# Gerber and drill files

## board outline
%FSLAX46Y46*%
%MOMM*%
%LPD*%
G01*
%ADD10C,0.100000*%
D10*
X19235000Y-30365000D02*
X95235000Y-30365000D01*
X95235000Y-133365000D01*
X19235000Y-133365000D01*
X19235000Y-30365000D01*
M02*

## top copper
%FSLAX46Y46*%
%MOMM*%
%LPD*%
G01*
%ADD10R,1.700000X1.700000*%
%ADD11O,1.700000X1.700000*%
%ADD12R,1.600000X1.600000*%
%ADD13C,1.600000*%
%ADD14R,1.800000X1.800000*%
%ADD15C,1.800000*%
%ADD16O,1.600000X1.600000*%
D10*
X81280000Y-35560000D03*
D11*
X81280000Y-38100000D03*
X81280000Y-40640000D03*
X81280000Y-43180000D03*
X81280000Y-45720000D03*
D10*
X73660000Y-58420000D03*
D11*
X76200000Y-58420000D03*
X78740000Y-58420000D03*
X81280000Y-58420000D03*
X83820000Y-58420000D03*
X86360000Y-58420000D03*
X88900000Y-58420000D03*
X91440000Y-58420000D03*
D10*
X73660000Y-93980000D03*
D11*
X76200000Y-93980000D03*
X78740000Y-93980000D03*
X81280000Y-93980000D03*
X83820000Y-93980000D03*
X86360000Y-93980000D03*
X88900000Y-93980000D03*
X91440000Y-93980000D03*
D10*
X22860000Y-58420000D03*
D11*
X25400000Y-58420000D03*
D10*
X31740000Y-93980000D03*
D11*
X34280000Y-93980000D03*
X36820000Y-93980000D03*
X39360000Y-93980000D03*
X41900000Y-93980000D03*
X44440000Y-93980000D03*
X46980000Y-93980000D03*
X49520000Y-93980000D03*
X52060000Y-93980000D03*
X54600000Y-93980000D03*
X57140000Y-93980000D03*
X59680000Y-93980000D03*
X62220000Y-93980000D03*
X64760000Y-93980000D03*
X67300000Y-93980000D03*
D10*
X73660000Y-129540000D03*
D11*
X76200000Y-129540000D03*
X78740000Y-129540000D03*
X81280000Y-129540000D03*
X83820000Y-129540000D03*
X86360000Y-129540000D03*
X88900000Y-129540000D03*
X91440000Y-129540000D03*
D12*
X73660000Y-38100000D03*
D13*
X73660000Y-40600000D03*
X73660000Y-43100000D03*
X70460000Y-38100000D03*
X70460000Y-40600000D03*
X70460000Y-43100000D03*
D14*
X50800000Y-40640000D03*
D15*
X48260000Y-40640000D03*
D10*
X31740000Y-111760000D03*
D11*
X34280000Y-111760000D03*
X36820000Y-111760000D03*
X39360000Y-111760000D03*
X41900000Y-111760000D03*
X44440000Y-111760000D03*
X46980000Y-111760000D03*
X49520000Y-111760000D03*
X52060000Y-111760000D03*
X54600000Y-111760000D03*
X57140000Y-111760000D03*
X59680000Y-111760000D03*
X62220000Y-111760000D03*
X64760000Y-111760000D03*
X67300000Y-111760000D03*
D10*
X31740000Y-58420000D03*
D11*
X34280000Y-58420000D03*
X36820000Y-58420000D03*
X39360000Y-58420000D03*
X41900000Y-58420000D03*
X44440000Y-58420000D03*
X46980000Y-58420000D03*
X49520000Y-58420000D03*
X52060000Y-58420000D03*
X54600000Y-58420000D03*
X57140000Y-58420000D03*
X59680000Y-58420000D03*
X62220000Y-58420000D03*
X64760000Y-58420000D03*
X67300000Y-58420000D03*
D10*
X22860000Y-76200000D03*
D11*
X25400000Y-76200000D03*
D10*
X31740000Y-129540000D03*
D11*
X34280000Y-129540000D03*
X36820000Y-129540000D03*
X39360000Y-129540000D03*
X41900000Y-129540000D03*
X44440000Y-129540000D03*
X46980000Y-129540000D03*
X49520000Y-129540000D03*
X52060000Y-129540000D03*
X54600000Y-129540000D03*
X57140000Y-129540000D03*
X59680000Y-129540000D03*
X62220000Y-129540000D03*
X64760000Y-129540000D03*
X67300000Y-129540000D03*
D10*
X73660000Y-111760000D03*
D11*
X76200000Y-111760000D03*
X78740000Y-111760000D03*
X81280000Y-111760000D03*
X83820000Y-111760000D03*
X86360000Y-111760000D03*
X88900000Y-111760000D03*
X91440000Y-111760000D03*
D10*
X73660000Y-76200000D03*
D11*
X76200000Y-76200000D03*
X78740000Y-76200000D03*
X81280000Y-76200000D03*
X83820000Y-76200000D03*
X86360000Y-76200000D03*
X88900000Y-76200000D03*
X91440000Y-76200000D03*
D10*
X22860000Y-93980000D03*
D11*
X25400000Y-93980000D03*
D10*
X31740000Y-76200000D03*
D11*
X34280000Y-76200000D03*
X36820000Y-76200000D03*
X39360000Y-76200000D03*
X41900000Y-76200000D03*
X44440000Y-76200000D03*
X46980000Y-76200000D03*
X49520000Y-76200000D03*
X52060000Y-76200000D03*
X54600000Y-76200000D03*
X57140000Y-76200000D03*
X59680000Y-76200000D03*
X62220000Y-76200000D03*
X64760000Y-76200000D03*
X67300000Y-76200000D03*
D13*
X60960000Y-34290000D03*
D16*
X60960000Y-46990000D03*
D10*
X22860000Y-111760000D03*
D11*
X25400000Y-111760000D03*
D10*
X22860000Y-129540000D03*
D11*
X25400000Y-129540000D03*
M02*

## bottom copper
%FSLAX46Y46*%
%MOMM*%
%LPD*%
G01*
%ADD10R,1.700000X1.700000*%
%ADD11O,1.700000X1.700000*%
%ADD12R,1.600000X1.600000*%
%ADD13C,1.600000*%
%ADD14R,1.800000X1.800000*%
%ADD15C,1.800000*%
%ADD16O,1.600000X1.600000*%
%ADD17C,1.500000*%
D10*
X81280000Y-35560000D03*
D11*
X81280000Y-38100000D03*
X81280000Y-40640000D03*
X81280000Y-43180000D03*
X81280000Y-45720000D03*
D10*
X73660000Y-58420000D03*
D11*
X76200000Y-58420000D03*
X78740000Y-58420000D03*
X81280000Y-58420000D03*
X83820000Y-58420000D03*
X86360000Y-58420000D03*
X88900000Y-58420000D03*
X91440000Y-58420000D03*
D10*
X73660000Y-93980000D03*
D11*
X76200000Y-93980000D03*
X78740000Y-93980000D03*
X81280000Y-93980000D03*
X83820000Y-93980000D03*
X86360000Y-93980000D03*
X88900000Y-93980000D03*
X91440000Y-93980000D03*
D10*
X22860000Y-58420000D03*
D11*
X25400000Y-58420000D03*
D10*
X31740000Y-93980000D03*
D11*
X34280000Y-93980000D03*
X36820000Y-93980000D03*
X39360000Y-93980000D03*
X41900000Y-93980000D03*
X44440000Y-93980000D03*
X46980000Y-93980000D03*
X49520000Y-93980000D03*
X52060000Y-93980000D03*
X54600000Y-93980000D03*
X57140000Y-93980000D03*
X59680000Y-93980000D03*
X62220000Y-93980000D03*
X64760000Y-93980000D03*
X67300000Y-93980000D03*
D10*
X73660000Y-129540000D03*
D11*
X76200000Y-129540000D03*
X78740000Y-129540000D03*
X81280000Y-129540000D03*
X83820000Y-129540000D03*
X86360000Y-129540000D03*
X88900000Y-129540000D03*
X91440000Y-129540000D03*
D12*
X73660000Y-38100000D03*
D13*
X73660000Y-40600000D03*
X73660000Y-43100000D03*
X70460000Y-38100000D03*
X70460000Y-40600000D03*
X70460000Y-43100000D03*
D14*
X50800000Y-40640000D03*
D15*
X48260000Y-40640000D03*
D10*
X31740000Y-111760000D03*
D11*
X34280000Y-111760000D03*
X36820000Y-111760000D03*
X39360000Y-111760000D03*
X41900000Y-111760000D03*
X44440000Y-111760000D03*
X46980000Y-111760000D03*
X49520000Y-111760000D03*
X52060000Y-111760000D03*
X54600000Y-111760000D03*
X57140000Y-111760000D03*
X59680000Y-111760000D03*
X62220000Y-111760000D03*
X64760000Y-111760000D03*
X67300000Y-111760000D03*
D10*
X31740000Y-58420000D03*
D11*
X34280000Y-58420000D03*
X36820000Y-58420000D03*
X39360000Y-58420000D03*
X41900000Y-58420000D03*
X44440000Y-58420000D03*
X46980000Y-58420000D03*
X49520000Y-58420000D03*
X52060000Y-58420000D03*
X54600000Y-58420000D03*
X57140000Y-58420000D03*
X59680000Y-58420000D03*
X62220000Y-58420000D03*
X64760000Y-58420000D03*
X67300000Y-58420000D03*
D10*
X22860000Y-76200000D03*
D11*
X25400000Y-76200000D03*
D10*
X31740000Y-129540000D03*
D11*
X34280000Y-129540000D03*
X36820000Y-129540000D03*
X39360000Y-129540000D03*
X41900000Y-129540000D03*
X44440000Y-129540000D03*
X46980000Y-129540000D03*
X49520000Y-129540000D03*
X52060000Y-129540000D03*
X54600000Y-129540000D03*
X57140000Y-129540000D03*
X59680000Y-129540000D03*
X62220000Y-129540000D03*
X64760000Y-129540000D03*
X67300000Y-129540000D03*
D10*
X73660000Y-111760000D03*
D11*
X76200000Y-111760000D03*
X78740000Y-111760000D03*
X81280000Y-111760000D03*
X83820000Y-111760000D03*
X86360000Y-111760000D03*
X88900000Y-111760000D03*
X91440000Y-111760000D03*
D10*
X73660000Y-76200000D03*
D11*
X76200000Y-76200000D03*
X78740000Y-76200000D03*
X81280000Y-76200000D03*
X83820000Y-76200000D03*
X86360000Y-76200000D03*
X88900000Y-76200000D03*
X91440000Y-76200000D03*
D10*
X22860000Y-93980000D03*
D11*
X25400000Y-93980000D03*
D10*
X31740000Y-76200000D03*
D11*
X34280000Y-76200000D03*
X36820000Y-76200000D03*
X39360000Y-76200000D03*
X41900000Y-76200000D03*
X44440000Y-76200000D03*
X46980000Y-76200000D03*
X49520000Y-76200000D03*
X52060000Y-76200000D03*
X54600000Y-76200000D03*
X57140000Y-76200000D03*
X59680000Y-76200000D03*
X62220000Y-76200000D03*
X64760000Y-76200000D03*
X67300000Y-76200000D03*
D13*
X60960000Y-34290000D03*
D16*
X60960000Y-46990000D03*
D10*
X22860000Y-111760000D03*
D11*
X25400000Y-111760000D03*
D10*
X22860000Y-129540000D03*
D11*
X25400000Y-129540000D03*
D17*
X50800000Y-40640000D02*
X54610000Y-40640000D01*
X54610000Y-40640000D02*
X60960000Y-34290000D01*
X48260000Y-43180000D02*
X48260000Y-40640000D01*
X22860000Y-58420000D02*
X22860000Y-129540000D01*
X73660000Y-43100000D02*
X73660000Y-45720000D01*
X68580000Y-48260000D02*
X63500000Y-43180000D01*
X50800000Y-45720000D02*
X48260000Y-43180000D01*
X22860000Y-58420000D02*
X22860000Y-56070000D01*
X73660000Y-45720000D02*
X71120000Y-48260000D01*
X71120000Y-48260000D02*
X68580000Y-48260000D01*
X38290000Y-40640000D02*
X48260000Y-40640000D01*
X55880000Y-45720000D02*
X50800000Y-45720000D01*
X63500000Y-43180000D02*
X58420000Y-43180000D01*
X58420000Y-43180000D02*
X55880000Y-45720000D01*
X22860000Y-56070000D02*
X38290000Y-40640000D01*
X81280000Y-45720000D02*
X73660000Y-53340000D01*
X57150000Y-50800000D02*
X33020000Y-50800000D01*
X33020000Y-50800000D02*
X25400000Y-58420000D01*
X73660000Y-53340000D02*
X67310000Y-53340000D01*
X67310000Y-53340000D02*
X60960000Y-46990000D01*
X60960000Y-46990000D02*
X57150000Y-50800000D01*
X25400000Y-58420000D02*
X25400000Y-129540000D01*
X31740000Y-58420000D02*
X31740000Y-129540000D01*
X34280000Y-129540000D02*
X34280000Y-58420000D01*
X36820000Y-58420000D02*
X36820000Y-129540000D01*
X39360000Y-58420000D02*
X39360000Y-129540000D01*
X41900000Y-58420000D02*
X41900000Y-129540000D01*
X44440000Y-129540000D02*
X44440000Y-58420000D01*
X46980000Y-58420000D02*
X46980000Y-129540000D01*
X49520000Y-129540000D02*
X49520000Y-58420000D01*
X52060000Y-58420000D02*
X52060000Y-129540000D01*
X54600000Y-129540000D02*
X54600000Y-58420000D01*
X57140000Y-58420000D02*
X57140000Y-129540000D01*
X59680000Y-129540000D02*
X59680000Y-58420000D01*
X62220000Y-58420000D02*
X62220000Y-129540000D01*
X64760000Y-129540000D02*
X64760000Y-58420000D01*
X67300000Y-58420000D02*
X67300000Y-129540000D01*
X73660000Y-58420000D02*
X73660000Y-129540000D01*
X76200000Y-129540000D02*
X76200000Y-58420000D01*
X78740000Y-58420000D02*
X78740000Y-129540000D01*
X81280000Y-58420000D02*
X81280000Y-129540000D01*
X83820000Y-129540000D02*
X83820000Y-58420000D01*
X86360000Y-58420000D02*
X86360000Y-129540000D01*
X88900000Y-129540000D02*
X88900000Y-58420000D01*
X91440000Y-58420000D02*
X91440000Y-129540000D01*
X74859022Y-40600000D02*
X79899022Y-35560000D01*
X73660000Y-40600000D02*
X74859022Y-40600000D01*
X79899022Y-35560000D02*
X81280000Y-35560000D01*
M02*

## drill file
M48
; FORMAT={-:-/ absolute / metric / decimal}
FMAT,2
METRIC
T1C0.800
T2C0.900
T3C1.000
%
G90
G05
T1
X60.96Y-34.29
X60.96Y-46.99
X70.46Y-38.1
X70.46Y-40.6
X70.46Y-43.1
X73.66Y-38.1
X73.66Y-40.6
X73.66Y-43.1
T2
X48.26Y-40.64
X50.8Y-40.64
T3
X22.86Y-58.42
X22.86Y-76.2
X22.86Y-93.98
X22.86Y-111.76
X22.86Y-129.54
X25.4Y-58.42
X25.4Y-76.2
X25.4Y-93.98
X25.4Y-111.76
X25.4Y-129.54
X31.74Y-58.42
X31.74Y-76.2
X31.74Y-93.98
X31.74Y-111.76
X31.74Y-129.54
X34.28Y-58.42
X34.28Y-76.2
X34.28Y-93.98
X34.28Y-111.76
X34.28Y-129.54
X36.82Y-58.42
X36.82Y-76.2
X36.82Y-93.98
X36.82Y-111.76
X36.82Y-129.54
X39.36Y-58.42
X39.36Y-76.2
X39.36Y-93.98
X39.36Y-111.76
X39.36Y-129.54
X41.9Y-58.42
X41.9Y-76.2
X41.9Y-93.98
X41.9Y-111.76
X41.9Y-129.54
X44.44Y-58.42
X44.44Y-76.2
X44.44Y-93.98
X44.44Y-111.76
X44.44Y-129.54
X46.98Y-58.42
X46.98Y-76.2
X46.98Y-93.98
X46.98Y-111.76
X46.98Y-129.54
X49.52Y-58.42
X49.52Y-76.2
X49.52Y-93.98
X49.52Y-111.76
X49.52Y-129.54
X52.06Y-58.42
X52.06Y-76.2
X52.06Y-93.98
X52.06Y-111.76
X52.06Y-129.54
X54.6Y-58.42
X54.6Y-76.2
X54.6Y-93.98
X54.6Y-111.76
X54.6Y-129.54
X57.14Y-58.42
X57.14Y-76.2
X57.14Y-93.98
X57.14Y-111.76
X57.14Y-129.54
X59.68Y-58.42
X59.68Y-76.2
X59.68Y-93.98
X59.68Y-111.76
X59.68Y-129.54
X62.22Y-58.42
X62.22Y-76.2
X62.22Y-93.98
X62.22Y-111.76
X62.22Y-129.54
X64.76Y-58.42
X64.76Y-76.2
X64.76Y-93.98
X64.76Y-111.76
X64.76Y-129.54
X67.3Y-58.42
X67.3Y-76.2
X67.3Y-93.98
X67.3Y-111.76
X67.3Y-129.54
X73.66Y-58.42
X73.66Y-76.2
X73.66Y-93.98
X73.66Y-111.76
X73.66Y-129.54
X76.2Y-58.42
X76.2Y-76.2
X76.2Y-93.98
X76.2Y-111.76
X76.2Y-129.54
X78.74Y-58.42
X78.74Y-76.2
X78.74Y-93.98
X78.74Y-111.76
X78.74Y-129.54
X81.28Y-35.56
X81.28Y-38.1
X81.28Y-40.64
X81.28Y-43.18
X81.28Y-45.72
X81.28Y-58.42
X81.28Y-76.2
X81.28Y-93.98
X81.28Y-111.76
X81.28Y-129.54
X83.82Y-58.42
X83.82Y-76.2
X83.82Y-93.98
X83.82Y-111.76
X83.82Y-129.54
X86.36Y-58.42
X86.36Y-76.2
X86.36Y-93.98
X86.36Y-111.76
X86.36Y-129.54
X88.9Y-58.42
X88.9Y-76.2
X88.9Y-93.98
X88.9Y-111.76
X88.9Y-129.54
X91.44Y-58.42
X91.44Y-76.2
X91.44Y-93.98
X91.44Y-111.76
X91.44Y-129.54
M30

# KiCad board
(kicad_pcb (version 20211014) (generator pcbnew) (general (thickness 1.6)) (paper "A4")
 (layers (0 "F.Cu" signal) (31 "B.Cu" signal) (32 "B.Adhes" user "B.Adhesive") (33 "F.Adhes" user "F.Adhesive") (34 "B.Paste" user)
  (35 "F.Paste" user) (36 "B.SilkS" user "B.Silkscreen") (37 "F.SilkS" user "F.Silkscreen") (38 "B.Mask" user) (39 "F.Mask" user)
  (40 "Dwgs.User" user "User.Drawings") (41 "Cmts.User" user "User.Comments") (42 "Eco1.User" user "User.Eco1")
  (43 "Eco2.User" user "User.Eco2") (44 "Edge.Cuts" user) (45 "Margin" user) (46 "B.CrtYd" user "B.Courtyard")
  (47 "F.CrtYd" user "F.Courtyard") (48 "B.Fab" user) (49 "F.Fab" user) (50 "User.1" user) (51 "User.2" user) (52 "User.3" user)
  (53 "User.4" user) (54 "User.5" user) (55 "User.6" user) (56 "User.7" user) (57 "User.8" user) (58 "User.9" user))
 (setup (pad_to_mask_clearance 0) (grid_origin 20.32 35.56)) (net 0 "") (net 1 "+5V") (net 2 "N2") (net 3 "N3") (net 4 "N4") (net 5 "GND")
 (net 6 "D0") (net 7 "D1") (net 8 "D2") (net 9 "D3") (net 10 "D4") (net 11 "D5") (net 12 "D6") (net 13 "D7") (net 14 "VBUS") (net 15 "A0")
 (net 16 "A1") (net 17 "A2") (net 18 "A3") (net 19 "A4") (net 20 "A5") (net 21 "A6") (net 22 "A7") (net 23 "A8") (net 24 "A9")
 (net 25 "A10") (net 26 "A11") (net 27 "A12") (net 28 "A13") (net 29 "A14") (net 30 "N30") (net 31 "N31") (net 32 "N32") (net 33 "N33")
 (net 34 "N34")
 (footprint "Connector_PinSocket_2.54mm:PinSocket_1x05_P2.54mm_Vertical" (layer "F.Cu") (at 81.28 35.56)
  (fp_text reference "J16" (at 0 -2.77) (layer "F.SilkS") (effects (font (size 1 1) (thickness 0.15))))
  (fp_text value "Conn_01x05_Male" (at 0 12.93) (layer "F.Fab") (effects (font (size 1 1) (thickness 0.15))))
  (pad "1" thru_hole rect locked (at 0 0) (size 1.7 1.7) (drill 1) (layers *.Cu *.Mask) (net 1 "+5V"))
  (pad "2" thru_hole oval locked (at 0 2.54) (size 1.7 1.7) (drill 1) (layers *.Cu *.Mask) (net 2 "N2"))
  (pad "3" thru_hole oval locked (at 0 5.08) (size 1.7 1.7) (drill 1) (layers *.Cu *.Mask) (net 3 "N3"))
  (pad "4" thru_hole oval locked (at 0 7.62) (size 1.7 1.7) (drill 1) (layers *.Cu *.Mask) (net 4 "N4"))
  (pad "5" thru_hole oval locked (at 0 10.16) (size 1.7 1.7) (drill 1) (layers *.Cu *.Mask) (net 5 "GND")))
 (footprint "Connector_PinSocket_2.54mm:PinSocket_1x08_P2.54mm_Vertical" (layer "F.Cu") (at 73.66 58.42 90)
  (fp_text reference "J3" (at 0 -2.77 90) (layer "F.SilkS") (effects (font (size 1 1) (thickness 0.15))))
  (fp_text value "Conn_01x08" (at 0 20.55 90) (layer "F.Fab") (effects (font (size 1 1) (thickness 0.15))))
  (pad "1" thru_hole rect locked (at 0 0 90) (size 1.7 1.7) (drill 1) (layers *.Cu *.Mask) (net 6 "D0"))
  (pad "2" thru_hole oval locked (at 0 2.54 90) (size 1.7 1.7) (drill 1) (layers *.Cu *.Mask) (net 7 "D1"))
  (pad "3" thru_hole oval locked (at 0 5.08 90) (size 1.7 1.7) (drill 1) (layers *.Cu *.Mask) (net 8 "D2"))
  (pad "4" thru_hole oval locked (at 0 7.62 90) (size 1.7 1.7) (drill 1) (layers *.Cu *.Mask) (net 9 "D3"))
  (pad "5" thru_hole oval locked (at 0 10.16 90) (size 1.7 1.7) (drill 1) (layers *.Cu *.Mask) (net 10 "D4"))
  (pad "6" thru_hole oval locked (at 0 12.7 90) (size 1.7 1.7) (drill 1) (layers *.Cu *.Mask) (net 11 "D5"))
  (pad "7" thru_hole oval locked (at 0 15.24 90) (size 1.7 1.7) (drill 1) (layers *.Cu *.Mask) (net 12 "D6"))
  (pad "8" thru_hole oval locked (at 0 17.78 90) (size 1.7 1.7) (drill 1) (layers *.Cu *.Mask) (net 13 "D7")))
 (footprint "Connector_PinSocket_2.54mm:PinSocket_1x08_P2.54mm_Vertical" (layer "F.Cu") (at 73.66 93.98 90)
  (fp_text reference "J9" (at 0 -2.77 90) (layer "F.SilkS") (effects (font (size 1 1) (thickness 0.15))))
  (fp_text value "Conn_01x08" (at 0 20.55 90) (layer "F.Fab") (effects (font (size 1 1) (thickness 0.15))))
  (pad "1" thru_hole rect locked (at 0 0 90) (size 1.7 1.7) (drill 1) (layers *.Cu *.Mask) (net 6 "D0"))
  (pad "2" thru_hole oval locked (at 0 2.54 90) (size 1.7 1.7) (drill 1) (layers *.Cu *.Mask) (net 7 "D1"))
  (pad "3" thru_hole oval locked (at 0 5.08 90) (size 1.7 1.7) (drill 1) (layers *.Cu *.Mask) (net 8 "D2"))
  (pad "4" thru_hole oval locked (at 0 7.62 90) (size 1.7 1.7) (drill 1) (layers *.Cu *.Mask) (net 9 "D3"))
  (pad "5" thru_hole oval locked (at 0 10.16 90) (size 1.7 1.7) (drill 1) (layers *.Cu *.Mask) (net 10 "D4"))
  (pad "6" thru_hole oval locked (at 0 12.7 90) (size 1.7 1.7) (drill 1) (layers *.Cu *.Mask) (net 11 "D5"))
  (pad "7" thru_hole oval locked (at 0 15.24 90) (size 1.7 1.7) (drill 1) (layers *.Cu *.Mask) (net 12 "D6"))
  (pad "8" thru_hole oval locked (at 0 17.78 90) (size 1.7 1.7) (drill 1) (layers *.Cu *.Mask) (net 13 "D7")))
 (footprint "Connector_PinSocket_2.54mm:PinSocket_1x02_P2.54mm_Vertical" (layer "F.Cu") (at 22.86 58.42 90)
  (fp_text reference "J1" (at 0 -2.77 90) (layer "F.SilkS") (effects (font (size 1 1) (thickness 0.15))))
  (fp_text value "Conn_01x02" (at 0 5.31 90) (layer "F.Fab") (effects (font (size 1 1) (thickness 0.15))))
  (pad "1" thru_hole rect locked (at 0 0 90) (size 1.7 1.7) (drill 1) (layers *.Cu *.Mask) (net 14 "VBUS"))
  (pad "2" thru_hole oval locked (at 0 2.54 90) (size 1.7 1.7) (drill 1) (layers *.Cu *.Mask) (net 5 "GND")))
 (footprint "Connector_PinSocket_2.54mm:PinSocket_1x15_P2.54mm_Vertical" (layer "F.Cu") (at 31.74 93.98 90)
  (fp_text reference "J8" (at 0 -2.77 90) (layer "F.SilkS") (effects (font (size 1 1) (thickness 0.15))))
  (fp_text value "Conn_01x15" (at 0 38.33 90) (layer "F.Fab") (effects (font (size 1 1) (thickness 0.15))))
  (pad "1" thru_hole rect locked (at 0 0 90) (size 1.7 1.7) (drill 1) (layers *.Cu *.Mask) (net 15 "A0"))
  (pad "2" thru_hole oval locked (at 0 2.54 90) (size 1.7 1.7) (drill 1) (layers *.Cu *.Mask) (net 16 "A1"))
  (pad "3" thru_hole oval locked (at 0 5.08 90) (size 1.7 1.7) (drill 1) (layers *.Cu *.Mask) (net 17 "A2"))
  (pad "4" thru_hole oval locked (at 0 7.62 90) (size 1.7 1.7) (drill 1) (layers *.Cu *.Mask) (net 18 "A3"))
  (pad "5" thru_hole oval locked (at 0 10.16 90) (size 1.7 1.7) (drill 1) (layers *.Cu *.Mask) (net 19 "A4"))
  (pad "6" thru_hole oval locked (at 0 12.7 90) (size 1.7 1.7) (drill 1) (layers *.Cu *.Mask) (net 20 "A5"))
  (pad "7" thru_hole oval locked (at 0 15.24 90) (size 1.7 1.7) (drill 1) (layers *.Cu *.Mask) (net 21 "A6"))
  (pad "8" thru_hole oval locked (at 0 17.78 90) (size 1.7 1.7) (drill 1) (layers *.Cu *.Mask) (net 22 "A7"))
  (pad "9" thru_hole oval locked (at 0 20.32 90) (size 1.7 1.7) (drill 1) (layers *.Cu *.Mask) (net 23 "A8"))
  (pad "10" thru_hole oval locked (at 0 22.86 90) (size 1.7 1.7) (drill 1) (layers *.Cu *.Mask) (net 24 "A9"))
  (pad "11" thru_hole oval locked (at 0 25.4 90) (size 1.7 1.7) (drill 1) (layers *.Cu *.Mask) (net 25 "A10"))
  (pad "12" thru_hole oval locked (at 0 27.94 90) (size 1.7 1.7) (drill 1) (layers *.Cu *.Mask) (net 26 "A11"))
  (pad "13" thru_hole oval locked (at 0 30.48 90) (size 1.7 1.7) (drill 1) (layers *.Cu *.Mask) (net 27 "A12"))
  (pad "14" thru_hole oval locked (at 0 33.02 90) (size 1.7 1.7) (drill 1) (layers *.Cu *.Mask) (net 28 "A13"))
  (pad "15" thru_hole oval locked (at 0 35.56 90) (size 1.7 1.7) (drill 1) (layers *.Cu *.Mask) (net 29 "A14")))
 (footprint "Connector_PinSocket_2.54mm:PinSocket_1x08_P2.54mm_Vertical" (layer "F.Cu") (at 73.66 129.54 90)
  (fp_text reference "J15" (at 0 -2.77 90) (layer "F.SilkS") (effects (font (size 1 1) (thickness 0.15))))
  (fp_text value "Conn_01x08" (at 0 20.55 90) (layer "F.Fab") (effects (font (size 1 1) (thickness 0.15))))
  (pad "1" thru_hole rect locked (at 0 0 90) (size 1.7 1.7) (drill 1) (layers *.Cu *.Mask) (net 6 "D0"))
  (pad "2" thru_hole oval locked (at 0 2.54 90) (size 1.7 1.7) (drill 1) (layers *.Cu *.Mask) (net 7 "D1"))
  (pad "3" thru_hole oval locked (at 0 5.08 90) (size 1.7 1.7) (drill 1) (layers *.Cu *.Mask) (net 8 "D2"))
  (pad "4" thru_hole oval locked (at 0 7.62 90) (size 1.7 1.7) (drill 1) (layers *.Cu *.Mask) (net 9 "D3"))
  (pad "5" thru_hole oval locked (at 0 10.16 90) (size 1.7 1.7) (drill 1) (layers *.Cu *.Mask) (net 10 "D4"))
  (pad "6" thru_hole oval locked (at 0 12.7 90) (size 1.7 1.7) (drill 1) (layers *.Cu *.Mask) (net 11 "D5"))
  (pad "7" thru_hole oval locked (at 0 15.24 90) (size 1.7 1.7) (drill 1) (layers *.Cu *.Mask) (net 12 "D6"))
  (pad "8" thru_hole oval locked (at 0 17.78 90) (size 1.7 1.7) (drill 1) (layers *.Cu *.Mask) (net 13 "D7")))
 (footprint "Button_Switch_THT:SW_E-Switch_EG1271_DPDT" (layer "F.Cu") (at 73.66 38.1 -90)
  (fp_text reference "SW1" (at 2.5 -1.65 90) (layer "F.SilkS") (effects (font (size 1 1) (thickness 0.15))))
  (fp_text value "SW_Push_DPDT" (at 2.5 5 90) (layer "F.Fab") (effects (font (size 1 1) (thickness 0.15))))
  (pad "1" thru_hole rect locked (at 0 0 270) (size 1.6 1.6) (drill 0.8) (layers *.Cu *.Mask) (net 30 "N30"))
  (pad "2" thru_hole circle locked (at 2.5 0 270) (size 1.6 1.6) (drill 0.8) (layers *.Cu *.Mask) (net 1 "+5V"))
  (pad "3" thru_hole circle locked (at 5 0 270) (size 1.6 1.6) (drill 0.8) (layers *.Cu *.Mask) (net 14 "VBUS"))
  (pad "4" thru_hole circle locked (at 0 3.2 270) (size 1.6 1.6) (drill 0.8) (layers *.Cu *.Mask) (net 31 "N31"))
  (pad "5" thru_hole circle locked (at 2.5 3.2 270) (size 1.6 1.6) (drill 0.8) (layers *.Cu *.Mask) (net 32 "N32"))
  (pad "6" thru_hole circle locked (at 5 3.2 270) (size 1.6 1.6) (drill 0.8) (layers *.Cu *.Mask) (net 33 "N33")))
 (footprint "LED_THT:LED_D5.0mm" (layer "F.Cu") (at 50.8 40.64 180)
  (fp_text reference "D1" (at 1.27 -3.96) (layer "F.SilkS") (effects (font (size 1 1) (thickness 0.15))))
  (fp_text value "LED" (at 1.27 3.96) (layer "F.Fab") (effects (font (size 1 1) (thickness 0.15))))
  (pad "1" thru_hole rect locked (at 0 0 180) (size 1.8 1.8) (drill 0.9) (layers *.Cu *.Mask) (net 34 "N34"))
  (pad "2" thru_hole circle locked (at 2.54 0 180) (size 1.8 1.8) (drill 0.9) (layers *.Cu *.Mask) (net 14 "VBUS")))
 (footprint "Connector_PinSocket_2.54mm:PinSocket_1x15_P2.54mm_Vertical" (layer "F.Cu") (at 31.74 111.76 90)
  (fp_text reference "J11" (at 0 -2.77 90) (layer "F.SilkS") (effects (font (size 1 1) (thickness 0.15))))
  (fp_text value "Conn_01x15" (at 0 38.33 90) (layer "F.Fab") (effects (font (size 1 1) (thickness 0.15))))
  (pad "1" thru_hole rect locked (at 0 0 90) (size 1.7 1.7) (drill 1) (layers *.Cu *.Mask) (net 15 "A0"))
  (pad "2" thru_hole oval locked (at 0 2.54 90) (size 1.7 1.7) (drill 1) (layers *.Cu *.Mask) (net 16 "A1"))
  (pad "3" thru_hole oval locked (at 0 5.08 90) (size 1.7 1.7) (drill 1) (layers *.Cu *.Mask) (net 17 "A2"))
  (pad "4" thru_hole oval locked (at 0 7.62 90) (size 1.7 1.7) (drill 1) (layers *.Cu *.Mask) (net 18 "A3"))
  (pad "5" thru_hole oval locked (at 0 10.16 90) (size 1.7 1.7) (drill 1) (layers *.Cu *.Mask) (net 19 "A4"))
  (pad "6" thru_hole oval locked (at 0 12.7 90) (size 1.7 1.7) (drill 1) (layers *.Cu *.Mask) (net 20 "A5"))
  (pad "7" thru_hole oval locked (at 0 15.24 90) (size 1.7 1.7) (drill 1) (layers *.Cu *.Mask) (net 21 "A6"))
  (pad "8" thru_hole oval locked (at 0 17.78 90) (size 1.7 1.7) (drill 1) (layers *.Cu *.Mask) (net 22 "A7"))
  (pad "9" thru_hole oval locked (at 0 20.32 90) (size 1.7 1.7) (drill 1) (layers *.Cu *.Mask) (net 23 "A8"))
  (pad "10" thru_hole oval locked (at 0 22.86 90) (size 1.7 1.7) (drill 1) (layers *.Cu *.Mask) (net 24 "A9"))
  (pad "11" thru_hole oval locked (at 0 25.4 90) (size 1.7 1.7) (drill 1) (layers *.Cu *.Mask) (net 25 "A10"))
  (pad "12" thru_hole oval locked (at 0 27.94 90) (size 1.7 1.7) (drill 1) (layers *.Cu *.Mask) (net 26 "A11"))
  (pad "13" thru_hole oval locked (at 0 30.48 90) (size 1.7 1.7) (drill 1) (layers *.Cu *.Mask) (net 27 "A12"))
  (pad "14" thru_hole oval locked (at 0 33.02 90) (size 1.7 1.7) (drill 1) (layers *.Cu *.Mask) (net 28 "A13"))
  (pad "15" thru_hole oval locked (at 0 35.56 90) (size 1.7 1.7) (drill 1) (layers *.Cu *.Mask) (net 29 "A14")))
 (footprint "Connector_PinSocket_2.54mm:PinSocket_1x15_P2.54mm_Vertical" (layer "F.Cu") (at 31.74 58.42 90)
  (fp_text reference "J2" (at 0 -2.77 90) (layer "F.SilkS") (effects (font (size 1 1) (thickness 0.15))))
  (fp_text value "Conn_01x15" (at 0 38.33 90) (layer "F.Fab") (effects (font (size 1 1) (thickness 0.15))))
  (pad "1" thru_hole rect locked (at 0 0 90) (size 1.7 1.7) (drill 1) (layers *.Cu *.Mask) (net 15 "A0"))
  (pad "2" thru_hole oval locked (at 0 2.54 90) (size 1.7 1.7) (drill 1) (layers *.Cu *.Mask) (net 16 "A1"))
  (pad "3" thru_hole oval locked (at 0 5.08 90) (size 1.7 1.7) (drill 1) (layers *.Cu *.Mask) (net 17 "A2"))
  (pad "4" thru_hole oval locked (at 0 7.62 90) (size 1.7 1.7) (drill 1) (layers *.Cu *.Mask) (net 18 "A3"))
  (pad "5" thru_hole oval locked (at 0 10.16 90) (size 1.7 1.7) (drill 1) (layers *.Cu *.Mask) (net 19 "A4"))
  (pad "6" thru_hole oval locked (at 0 12.7 90) (size 1.7 1.7) (drill 1) (layers *.Cu *.Mask) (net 20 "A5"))
  (pad "7" thru_hole oval locked (at 0 15.24 90) (size 1.7 1.7) (drill 1) (layers *.Cu *.Mask) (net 21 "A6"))
  (pad "8" thru_hole oval locked (at 0 17.78 90) (size 1.7 1.7) (drill 1) (layers *.Cu *.Mask) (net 22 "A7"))
  (pad "9" thru_hole oval locked (at 0 20.32 90) (size 1.7 1.7) (drill 1) (layers *.Cu *.Mask) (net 23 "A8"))
  (pad "10" thru_hole oval locked (at 0 22.86 90) (size 1.7 1.7) (drill 1) (layers *.Cu *.Mask) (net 24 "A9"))
  (pad "11" thru_hole oval locked (at 0 25.4 90) (size 1.7 1.7) (drill 1) (layers *.Cu *.Mask) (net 25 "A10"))
  (pad "12" thru_hole oval locked (at 0 27.94 90) (size 1.7 1.7) (drill 1) (layers *.Cu *.Mask) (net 26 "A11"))
  (pad "13" thru_hole oval locked (at 0 30.48 90) (size 1.7 1.7) (drill 1) (layers *.Cu *.Mask) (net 27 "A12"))
  (pad "14" thru_hole oval locked (at 0 33.02 90) (size 1.7 1.7) (drill 1) (layers *.Cu *.Mask) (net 28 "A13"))
  (pad "15" thru_hole oval locked (at 0 35.56 90) (size 1.7 1.7) (drill 1) (layers *.Cu *.Mask) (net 29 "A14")))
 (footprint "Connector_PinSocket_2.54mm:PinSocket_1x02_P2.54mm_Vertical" (layer "F.Cu") (at 22.86 76.2 90)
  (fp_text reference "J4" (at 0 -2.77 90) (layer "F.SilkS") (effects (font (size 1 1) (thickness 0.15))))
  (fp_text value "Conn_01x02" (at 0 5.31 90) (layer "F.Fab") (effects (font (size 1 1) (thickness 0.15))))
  (pad "1" thru_hole rect locked (at 0 0 90) (size 1.7 1.7) (drill 1) (layers *.Cu *.Mask) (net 14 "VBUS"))
  (pad "2" thru_hole oval locked (at 0 2.54 90) (size 1.7 1.7) (drill 1) (layers *.Cu *.Mask) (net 5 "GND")))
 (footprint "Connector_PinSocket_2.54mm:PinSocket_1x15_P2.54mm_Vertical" (layer "F.Cu") (at 31.74 129.54 90)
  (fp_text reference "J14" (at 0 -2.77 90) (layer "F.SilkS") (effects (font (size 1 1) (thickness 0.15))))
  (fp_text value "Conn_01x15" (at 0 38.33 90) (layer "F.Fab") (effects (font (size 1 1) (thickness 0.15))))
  (pad "1" thru_hole rect locked (at 0 0 90) (size 1.7 1.7) (drill 1) (layers *.Cu *.Mask) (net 15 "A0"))
  (pad "2" thru_hole oval locked (at 0 2.54 90) (size 1.7 1.7) (drill 1) (layers *.Cu *.Mask) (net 16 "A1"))
  (pad "3" thru_hole oval locked (at 0 5.08 90) (size 1.7 1.7) (drill 1) (layers *.Cu *.Mask) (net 17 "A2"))
  (pad "4" thru_hole oval locked (at 0 7.62 90) (size 1.7 1.7) (drill 1) (layers *.Cu *.Mask) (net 18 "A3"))
  (pad "5" thru_hole oval locked (at 0 10.16 90) (size 1.7 1.7) (drill 1) (layers *.Cu *.Mask) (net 19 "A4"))
  (pad "6" thru_hole oval locked (at 0 12.7 90) (size 1.7 1.7) (drill 1) (layers *.Cu *.Mask) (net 20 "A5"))
  (pad "7" thru_hole oval locked (at 0 15.24 90) (size 1.7 1.7) (drill 1) (layers *.Cu *.Mask) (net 21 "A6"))
  (pad "8" thru_hole oval locked (at 0 17.78 90) (size 1.7 1.7) (drill 1) (layers *.Cu *.Mask) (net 22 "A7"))
  (pad "9" thru_hole oval locked (at 0 20.32 90) (size 1.7 1.7) (drill 1) (layers *.Cu *.Mask) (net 23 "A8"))
  (pad "10" thru_hole oval locked (at 0 22.86 90) (size 1.7 1.7) (drill 1) (layers *.Cu *.Mask) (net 24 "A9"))
  (pad "11" thru_hole oval locked (at 0 25.4 90) (size 1.7 1.7) (drill 1) (layers *.Cu *.Mask) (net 25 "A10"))
  (pad "12" thru_hole oval locked (at 0 27.94 90) (size 1.7 1.7) (drill 1) (layers *.Cu *.Mask) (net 26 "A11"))
  (pad "13" thru_hole oval locked (at 0 30.48 90) (size 1.7 1.7) (drill 1) (layers *.Cu *.Mask) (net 27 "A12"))
  (pad "14" thru_hole oval locked (at 0 33.02 90) (size 1.7 1.7) (drill 1) (layers *.Cu *.Mask) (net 28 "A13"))
  (pad "15" thru_hole oval locked (at 0 35.56 90) (size 1.7 1.7) (drill 1) (layers *.Cu *.Mask) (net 29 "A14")))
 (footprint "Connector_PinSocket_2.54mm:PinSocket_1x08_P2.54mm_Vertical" (layer "F.Cu") (at 73.66 111.76 90)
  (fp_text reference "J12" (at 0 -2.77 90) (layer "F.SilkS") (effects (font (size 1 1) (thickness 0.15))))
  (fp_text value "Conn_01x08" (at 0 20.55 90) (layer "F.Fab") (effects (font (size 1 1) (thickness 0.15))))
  (pad "1" thru_hole rect locked (at 0 0 90) (size 1.7 1.7) (drill 1) (layers *.Cu *.Mask) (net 6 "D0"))
  (pad "2" thru_hole oval locked (at 0 2.54 90) (size 1.7 1.7) (drill 1) (layers *.Cu *.Mask) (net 7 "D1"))
  (pad "3" thru_hole oval locked (at 0 5.08 90) (size 1.7 1.7) (drill 1) (layers *.Cu *.Mask) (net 8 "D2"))
  (pad "4" thru_hole oval locked (at 0 7.62 90) (size 1.7 1.7) (drill 1) (layers *.Cu *.Mask) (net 9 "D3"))
  (pad "5" thru_hole oval locked (at 0 10.16 90) (size 1.7 1.7) (drill 1) (layers *.Cu *.Mask) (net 10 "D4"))
  (pad "6" thru_hole oval locked (at 0 12.7 90) (size 1.7 1.7) (drill 1) (layers *.Cu *.Mask) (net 11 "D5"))
  (pad "7" thru_hole oval locked (at 0 15.24 90) (size 1.7 1.7) (drill 1) (layers *.Cu *.Mask) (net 12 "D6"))
  (pad "8" thru_hole oval locked (at 0 17.78 90) (size 1.7 1.7) (drill 1) (layers *.Cu *.Mask) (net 13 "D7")))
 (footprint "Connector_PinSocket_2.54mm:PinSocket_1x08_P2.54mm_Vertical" (layer "F.Cu") (at 73.66 76.2 90)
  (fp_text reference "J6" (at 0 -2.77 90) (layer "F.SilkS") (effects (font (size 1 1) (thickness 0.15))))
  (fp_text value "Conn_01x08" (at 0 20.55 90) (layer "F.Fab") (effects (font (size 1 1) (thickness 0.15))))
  (pad "1" thru_hole rect locked (at 0 0 90) (size 1.7 1.7) (drill 1) (layers *.Cu *.Mask) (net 6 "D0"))
  (pad "2" thru_hole oval locked (at 0 2.54 90) (size 1.7 1.7) (drill 1) (layers *.Cu *.Mask) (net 7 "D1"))
  (pad "3" thru_hole oval locked (at 0 5.08 90) (size 1.7 1.7) (drill 1) (layers *.Cu *.Mask) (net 8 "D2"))
  (pad "4" thru_hole oval locked (at 0 7.62 90) (size 1.7 1.7) (drill 1) (layers *.Cu *.Mask) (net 9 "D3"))
  (pad "5" thru_hole oval locked (at 0 10.16 90) (size 1.7 1.7) (drill 1) (layers *.Cu *.Mask) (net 10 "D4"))
  (pad "6" thru_hole oval locked (at 0 12.7 90) (size 1.7 1.7) (drill 1) (layers *.Cu *.Mask) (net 11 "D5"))
  (pad "7" thru_hole oval locked (at 0 15.24 90) (size 1.7 1.7) (drill 1) (layers *.Cu *.Mask) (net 12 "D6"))
  (pad "8" thru_hole oval locked (at 0 17.78 90) (size 1.7 1.7) (drill 1) (layers *.Cu *.Mask) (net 13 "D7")))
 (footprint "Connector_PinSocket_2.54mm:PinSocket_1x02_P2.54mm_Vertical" (layer "F.Cu") (at 22.86 93.98 90)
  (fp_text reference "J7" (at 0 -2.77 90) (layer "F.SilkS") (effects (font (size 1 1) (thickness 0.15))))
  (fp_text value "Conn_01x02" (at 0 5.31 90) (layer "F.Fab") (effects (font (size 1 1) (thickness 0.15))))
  (pad "1" thru_hole rect locked (at 0 0 90) (size 1.7 1.7) (drill 1) (layers *.Cu *.Mask) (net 14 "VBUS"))
  (pad "2" thru_hole oval locked (at 0 2.54 90) (size 1.7 1.7) (drill 1) (layers *.Cu *.Mask) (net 5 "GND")))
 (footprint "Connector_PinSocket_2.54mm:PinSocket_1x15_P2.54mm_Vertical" (layer "F.Cu") (at 31.74 76.2 90)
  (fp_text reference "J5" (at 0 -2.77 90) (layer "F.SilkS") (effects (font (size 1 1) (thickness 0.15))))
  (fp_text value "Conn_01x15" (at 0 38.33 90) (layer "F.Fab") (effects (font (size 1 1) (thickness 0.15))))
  (pad "1" thru_hole rect locked (at 0 0 90) (size 1.7 1.7) (drill 1) (layers *.Cu *.Mask) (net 15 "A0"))
  (pad "2" thru_hole oval locked (at 0 2.54 90) (size 1.7 1.7) (drill 1) (layers *.Cu *.Mask) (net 16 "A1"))
  (pad "3" thru_hole oval locked (at 0 5.08 90) (size 1.7 1.7) (drill 1) (layers *.Cu *.Mask) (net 17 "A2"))
  (pad "4" thru_hole oval locked (at 0 7.62 90) (size 1.7 1.7) (drill 1) (layers *.Cu *.Mask) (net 18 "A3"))
  (pad "5" thru_hole oval locked (at 0 10.16 90) (size 1.7 1.7) (drill 1) (layers *.Cu *.Mask) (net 19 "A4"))
  (pad "6" thru_hole oval locked (at 0 12.7 90) (size 1.7 1.7) (drill 1) (layers *.Cu *.Mask) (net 20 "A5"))
  (pad "7" thru_hole oval locked (at 0 15.24 90) (size 1.7 1.7) (drill 1) (layers *.Cu *.Mask) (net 21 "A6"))
  (pad "8" thru_hole oval locked (at 0 17.78 90) (size 1.7 1.7) (drill 1) (layers *.Cu *.Mask) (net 22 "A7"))
  (pad "9" thru_hole oval locked (at 0 20.32 90) (size 1.7 1.7) (drill 1) (layers *.Cu *.Mask) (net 23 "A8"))
  (pad "10" thru_hole oval locked (at 0 22.86 90) (size 1.7 1.7) (drill 1) (layers *.Cu *.Mask) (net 24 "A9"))
  (pad "11" thru_hole oval locked (at 0 25.4 90) (size 1.7 1.7) (drill 1) (layers *.Cu *.Mask) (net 25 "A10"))
  (pad "12" thru_hole oval locked (at 0 27.94 90) (size 1.7 1.7) (drill 1) (layers *.Cu *.Mask) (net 26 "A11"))
  (pad "13" thru_hole oval locked (at 0 30.48 90) (size 1.7 1.7) (drill 1) (layers *.Cu *.Mask) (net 27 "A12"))
  (pad "14" thru_hole oval locked (at 0 33.02 90) (size 1.7 1.7) (drill 1) (layers *.Cu *.Mask) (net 28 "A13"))
  (pad "15" thru_hole oval locked (at 0 35.56 90) (size 1.7 1.7) (drill 1) (layers *.Cu *.Mask) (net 29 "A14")))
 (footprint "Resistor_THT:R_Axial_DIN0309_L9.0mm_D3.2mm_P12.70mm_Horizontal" (layer "F.Cu") (at 60.96 34.29 -90)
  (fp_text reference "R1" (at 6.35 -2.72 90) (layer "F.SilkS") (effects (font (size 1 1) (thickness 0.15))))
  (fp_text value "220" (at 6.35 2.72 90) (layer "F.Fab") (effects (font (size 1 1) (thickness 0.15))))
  (pad "1" thru_hole circle locked (at 0 0 270) (size 1.6 1.6) (drill 0.8) (layers *.Cu *.Mask) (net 34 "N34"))
  (pad "2" thru_hole oval locked (at 12.7 0 270) (size 1.6 1.6) (drill 0.8) (layers *.Cu *.Mask) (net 5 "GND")))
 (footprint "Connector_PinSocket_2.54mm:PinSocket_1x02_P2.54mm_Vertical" (layer "F.Cu") (at 22.86 111.76 90)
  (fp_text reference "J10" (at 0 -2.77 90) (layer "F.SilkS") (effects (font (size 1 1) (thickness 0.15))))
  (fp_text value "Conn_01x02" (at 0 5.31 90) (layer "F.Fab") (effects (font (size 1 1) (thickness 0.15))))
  (pad "1" thru_hole rect locked (at 0 0 90) (size 1.7 1.7) (drill 1) (layers *.Cu *.Mask) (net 14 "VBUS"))
  (pad "2" thru_hole oval locked (at 0 2.54 90) (size 1.7 1.7) (drill 1) (layers *.Cu *.Mask) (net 5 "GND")))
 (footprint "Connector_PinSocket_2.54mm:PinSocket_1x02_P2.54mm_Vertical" (layer "F.Cu") (at 22.86 129.54 90)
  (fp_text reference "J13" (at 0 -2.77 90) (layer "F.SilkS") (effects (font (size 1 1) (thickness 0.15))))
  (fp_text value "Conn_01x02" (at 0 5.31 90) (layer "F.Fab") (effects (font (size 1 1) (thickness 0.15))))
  (pad "1" thru_hole rect locked (at 0 0 90) (size 1.7 1.7) (drill 1) (layers *.Cu *.Mask) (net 14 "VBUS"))
  (pad "2" thru_hole oval locked (at 0 2.54 90) (size 1.7 1.7) (drill 1) (layers *.Cu *.Mask) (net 5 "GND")))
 (gr_rect (start 19.235 30.365) (end 95.235 133.365) (layer "Edge.Cuts") (width 0.1) (fill none))
 (segment (start 50.8 40.64) (end 54.61 40.64) (width 1.5) (layer "B.Cu") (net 34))
 (segment (start 54.61 40.64) (end 60.96 34.29) (width 1.5) (layer "B.Cu") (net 34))
 (segment (start 48.26 43.18) (end 48.26 40.64) (width 1.5) (layer "B.Cu") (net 14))
 (segment (start 22.86 58.42) (end 22.86 129.54) (width 1.5) (layer "B.Cu") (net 14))
 (segment (start 73.66 43.1) (end 73.66 45.72) (width 1.5) (layer "B.Cu") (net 14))
 (segment (start 68.58 48.26) (end 63.5 43.18) (width 1.5) (layer "B.Cu") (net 14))
 (segment (start 50.8 45.72) (end 48.26 43.18) (width 1.5) (layer "B.Cu") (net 14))
 (segment (start 22.86 58.42) (end 22.86 56.07) (width 1.5) (layer "B.Cu") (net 14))
 (segment (start 73.66 45.72) (end 71.12 48.26) (width 1.5) (layer "B.Cu") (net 14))
 (segment (start 71.12 48.26) (end 68.58 48.26) (width 1.5) (layer "B.Cu") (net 14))
 (segment (start 38.29 40.64) (end 48.26 40.64) (width 1.5) (layer "B.Cu") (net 14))
 (segment (start 55.88 45.72) (end 50.8 45.72) (width 1.5) (layer "B.Cu") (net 14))
 (segment (start 63.5 43.18) (end 58.42 43.18) (width 1.5) (layer "B.Cu") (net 14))
 (segment (start 58.42 43.18) (end 55.88 45.72) (width 1.5) (layer "B.Cu") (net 14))
 (segment (start 22.86 56.07) (end 38.29 40.64) (width 1.5) (layer "B.Cu") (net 14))
 (segment (start 81.28 45.72) (end 73.66 53.34) (width 1.5) (layer "B.Cu") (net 5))
 (segment (start 57.15 50.8) (end 33.02 50.8) (width 1.5) (layer "B.Cu") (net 5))
 (segment (start 33.02 50.8) (end 25.4 58.42) (width 1.5) (layer "B.Cu") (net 5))
 (segment (start 73.66 53.34) (end 67.31 53.34) (width 1.5) (layer "B.Cu") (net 5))
 (segment (start 67.31 53.34) (end 60.96 46.99) (width 1.5) (layer "B.Cu") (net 5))
 (segment (start 60.96 46.99) (end 57.15 50.8) (width 1.5) (layer "B.Cu") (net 5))
 (segment (start 25.4 58.42) (end 25.4 129.54) (width 1.5) (layer "B.Cu") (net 5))
 (segment (start 31.74 58.42) (end 31.74 129.54) (width 1.5) (layer "B.Cu") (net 15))
 (segment (start 34.28 129.54) (end 34.28 58.42) (width 1.5) (layer "B.Cu") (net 16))
 (segment (start 36.82 58.42) (end 36.82 129.54) (width 1.5) (layer "B.Cu") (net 17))
 (segment (start 39.36 58.42) (end 39.36 129.54) (width 1.5) (layer "B.Cu") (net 18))
 (segment (start 41.9 58.42) (end 41.9 129.54) (width 1.5) (layer "B.Cu") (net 19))
 (segment (start 44.44 129.54) (end 44.44 58.42) (width 1.5) (layer "B.Cu") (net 20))
 (segment (start 46.98 58.42) (end 46.98 129.54) (width 1.5) (layer "B.Cu") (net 21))
 (segment (start 49.52 129.54) (end 49.52 58.42) (width 1.5) (layer "B.Cu") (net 22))
 (segment (start 52.06 58.42) (end 52.06 129.54) (width 1.5) (layer "B.Cu") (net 23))
 (segment (start 54.6 129.54) (end 54.6 58.42) (width 1.5) (layer "B.Cu") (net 24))
 (segment (start 57.14 58.42) (end 57.14 129.54) (width 1.5) (layer "B.Cu") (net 25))
 (segment (start 59.68 129.54) (end 59.68 58.42) (width 1.5) (layer "B.Cu") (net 26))
 (segment (start 62.22 58.42) (end 62.22 129.54) (width 1.5) (layer "B.Cu") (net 27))
 (segment (start 64.76 129.54) (end 64.76 58.42) (width 1.5) (layer "B.Cu") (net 28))
 (segment (start 67.3 58.42) (end 67.3 129.54) (width 1.5) (layer "B.Cu") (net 29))
 (segment (start 73.66 58.42) (end 73.66 129.54) (width 1.5) (layer "B.Cu") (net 6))
 (segment (start 76.2 129.54) (end 76.2 58.42) (width 1.5) (layer "B.Cu") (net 7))
 (segment (start 78.74 58.42) (end 78.74 129.54) (width 1.5) (layer "B.Cu") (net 8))
 (segment (start 81.28 58.42) (end 81.28 129.54) (width 1.5) (layer "B.Cu") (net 9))
 (segment (start 83.82 129.54) (end 83.82 58.42) (width 1.5) (layer "B.Cu") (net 10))
 (segment (start 86.36 58.42) (end 86.36 129.54) (width 1.5) (layer "B.Cu") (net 11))
 (segment (start 88.9 129.54) (end 88.9 58.42) (width 1.5) (layer "B.Cu") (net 12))
 (segment (start 91.44 58.42) (end 91.44 129.54) (width 1.5) (layer "B.Cu") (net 13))
 (segment (start 74.859022 40.6) (end 79.899022 35.56) (width 1.5) (layer "B.Cu") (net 1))
 (segment (start 73.66 40.6) (end 74.859022 40.6) (width 1.5) (layer "B.Cu") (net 1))
 (segment (start 79.899022 35.56) (end 81.28 35.56) (width 1.5) (layer "B.Cu") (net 1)))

